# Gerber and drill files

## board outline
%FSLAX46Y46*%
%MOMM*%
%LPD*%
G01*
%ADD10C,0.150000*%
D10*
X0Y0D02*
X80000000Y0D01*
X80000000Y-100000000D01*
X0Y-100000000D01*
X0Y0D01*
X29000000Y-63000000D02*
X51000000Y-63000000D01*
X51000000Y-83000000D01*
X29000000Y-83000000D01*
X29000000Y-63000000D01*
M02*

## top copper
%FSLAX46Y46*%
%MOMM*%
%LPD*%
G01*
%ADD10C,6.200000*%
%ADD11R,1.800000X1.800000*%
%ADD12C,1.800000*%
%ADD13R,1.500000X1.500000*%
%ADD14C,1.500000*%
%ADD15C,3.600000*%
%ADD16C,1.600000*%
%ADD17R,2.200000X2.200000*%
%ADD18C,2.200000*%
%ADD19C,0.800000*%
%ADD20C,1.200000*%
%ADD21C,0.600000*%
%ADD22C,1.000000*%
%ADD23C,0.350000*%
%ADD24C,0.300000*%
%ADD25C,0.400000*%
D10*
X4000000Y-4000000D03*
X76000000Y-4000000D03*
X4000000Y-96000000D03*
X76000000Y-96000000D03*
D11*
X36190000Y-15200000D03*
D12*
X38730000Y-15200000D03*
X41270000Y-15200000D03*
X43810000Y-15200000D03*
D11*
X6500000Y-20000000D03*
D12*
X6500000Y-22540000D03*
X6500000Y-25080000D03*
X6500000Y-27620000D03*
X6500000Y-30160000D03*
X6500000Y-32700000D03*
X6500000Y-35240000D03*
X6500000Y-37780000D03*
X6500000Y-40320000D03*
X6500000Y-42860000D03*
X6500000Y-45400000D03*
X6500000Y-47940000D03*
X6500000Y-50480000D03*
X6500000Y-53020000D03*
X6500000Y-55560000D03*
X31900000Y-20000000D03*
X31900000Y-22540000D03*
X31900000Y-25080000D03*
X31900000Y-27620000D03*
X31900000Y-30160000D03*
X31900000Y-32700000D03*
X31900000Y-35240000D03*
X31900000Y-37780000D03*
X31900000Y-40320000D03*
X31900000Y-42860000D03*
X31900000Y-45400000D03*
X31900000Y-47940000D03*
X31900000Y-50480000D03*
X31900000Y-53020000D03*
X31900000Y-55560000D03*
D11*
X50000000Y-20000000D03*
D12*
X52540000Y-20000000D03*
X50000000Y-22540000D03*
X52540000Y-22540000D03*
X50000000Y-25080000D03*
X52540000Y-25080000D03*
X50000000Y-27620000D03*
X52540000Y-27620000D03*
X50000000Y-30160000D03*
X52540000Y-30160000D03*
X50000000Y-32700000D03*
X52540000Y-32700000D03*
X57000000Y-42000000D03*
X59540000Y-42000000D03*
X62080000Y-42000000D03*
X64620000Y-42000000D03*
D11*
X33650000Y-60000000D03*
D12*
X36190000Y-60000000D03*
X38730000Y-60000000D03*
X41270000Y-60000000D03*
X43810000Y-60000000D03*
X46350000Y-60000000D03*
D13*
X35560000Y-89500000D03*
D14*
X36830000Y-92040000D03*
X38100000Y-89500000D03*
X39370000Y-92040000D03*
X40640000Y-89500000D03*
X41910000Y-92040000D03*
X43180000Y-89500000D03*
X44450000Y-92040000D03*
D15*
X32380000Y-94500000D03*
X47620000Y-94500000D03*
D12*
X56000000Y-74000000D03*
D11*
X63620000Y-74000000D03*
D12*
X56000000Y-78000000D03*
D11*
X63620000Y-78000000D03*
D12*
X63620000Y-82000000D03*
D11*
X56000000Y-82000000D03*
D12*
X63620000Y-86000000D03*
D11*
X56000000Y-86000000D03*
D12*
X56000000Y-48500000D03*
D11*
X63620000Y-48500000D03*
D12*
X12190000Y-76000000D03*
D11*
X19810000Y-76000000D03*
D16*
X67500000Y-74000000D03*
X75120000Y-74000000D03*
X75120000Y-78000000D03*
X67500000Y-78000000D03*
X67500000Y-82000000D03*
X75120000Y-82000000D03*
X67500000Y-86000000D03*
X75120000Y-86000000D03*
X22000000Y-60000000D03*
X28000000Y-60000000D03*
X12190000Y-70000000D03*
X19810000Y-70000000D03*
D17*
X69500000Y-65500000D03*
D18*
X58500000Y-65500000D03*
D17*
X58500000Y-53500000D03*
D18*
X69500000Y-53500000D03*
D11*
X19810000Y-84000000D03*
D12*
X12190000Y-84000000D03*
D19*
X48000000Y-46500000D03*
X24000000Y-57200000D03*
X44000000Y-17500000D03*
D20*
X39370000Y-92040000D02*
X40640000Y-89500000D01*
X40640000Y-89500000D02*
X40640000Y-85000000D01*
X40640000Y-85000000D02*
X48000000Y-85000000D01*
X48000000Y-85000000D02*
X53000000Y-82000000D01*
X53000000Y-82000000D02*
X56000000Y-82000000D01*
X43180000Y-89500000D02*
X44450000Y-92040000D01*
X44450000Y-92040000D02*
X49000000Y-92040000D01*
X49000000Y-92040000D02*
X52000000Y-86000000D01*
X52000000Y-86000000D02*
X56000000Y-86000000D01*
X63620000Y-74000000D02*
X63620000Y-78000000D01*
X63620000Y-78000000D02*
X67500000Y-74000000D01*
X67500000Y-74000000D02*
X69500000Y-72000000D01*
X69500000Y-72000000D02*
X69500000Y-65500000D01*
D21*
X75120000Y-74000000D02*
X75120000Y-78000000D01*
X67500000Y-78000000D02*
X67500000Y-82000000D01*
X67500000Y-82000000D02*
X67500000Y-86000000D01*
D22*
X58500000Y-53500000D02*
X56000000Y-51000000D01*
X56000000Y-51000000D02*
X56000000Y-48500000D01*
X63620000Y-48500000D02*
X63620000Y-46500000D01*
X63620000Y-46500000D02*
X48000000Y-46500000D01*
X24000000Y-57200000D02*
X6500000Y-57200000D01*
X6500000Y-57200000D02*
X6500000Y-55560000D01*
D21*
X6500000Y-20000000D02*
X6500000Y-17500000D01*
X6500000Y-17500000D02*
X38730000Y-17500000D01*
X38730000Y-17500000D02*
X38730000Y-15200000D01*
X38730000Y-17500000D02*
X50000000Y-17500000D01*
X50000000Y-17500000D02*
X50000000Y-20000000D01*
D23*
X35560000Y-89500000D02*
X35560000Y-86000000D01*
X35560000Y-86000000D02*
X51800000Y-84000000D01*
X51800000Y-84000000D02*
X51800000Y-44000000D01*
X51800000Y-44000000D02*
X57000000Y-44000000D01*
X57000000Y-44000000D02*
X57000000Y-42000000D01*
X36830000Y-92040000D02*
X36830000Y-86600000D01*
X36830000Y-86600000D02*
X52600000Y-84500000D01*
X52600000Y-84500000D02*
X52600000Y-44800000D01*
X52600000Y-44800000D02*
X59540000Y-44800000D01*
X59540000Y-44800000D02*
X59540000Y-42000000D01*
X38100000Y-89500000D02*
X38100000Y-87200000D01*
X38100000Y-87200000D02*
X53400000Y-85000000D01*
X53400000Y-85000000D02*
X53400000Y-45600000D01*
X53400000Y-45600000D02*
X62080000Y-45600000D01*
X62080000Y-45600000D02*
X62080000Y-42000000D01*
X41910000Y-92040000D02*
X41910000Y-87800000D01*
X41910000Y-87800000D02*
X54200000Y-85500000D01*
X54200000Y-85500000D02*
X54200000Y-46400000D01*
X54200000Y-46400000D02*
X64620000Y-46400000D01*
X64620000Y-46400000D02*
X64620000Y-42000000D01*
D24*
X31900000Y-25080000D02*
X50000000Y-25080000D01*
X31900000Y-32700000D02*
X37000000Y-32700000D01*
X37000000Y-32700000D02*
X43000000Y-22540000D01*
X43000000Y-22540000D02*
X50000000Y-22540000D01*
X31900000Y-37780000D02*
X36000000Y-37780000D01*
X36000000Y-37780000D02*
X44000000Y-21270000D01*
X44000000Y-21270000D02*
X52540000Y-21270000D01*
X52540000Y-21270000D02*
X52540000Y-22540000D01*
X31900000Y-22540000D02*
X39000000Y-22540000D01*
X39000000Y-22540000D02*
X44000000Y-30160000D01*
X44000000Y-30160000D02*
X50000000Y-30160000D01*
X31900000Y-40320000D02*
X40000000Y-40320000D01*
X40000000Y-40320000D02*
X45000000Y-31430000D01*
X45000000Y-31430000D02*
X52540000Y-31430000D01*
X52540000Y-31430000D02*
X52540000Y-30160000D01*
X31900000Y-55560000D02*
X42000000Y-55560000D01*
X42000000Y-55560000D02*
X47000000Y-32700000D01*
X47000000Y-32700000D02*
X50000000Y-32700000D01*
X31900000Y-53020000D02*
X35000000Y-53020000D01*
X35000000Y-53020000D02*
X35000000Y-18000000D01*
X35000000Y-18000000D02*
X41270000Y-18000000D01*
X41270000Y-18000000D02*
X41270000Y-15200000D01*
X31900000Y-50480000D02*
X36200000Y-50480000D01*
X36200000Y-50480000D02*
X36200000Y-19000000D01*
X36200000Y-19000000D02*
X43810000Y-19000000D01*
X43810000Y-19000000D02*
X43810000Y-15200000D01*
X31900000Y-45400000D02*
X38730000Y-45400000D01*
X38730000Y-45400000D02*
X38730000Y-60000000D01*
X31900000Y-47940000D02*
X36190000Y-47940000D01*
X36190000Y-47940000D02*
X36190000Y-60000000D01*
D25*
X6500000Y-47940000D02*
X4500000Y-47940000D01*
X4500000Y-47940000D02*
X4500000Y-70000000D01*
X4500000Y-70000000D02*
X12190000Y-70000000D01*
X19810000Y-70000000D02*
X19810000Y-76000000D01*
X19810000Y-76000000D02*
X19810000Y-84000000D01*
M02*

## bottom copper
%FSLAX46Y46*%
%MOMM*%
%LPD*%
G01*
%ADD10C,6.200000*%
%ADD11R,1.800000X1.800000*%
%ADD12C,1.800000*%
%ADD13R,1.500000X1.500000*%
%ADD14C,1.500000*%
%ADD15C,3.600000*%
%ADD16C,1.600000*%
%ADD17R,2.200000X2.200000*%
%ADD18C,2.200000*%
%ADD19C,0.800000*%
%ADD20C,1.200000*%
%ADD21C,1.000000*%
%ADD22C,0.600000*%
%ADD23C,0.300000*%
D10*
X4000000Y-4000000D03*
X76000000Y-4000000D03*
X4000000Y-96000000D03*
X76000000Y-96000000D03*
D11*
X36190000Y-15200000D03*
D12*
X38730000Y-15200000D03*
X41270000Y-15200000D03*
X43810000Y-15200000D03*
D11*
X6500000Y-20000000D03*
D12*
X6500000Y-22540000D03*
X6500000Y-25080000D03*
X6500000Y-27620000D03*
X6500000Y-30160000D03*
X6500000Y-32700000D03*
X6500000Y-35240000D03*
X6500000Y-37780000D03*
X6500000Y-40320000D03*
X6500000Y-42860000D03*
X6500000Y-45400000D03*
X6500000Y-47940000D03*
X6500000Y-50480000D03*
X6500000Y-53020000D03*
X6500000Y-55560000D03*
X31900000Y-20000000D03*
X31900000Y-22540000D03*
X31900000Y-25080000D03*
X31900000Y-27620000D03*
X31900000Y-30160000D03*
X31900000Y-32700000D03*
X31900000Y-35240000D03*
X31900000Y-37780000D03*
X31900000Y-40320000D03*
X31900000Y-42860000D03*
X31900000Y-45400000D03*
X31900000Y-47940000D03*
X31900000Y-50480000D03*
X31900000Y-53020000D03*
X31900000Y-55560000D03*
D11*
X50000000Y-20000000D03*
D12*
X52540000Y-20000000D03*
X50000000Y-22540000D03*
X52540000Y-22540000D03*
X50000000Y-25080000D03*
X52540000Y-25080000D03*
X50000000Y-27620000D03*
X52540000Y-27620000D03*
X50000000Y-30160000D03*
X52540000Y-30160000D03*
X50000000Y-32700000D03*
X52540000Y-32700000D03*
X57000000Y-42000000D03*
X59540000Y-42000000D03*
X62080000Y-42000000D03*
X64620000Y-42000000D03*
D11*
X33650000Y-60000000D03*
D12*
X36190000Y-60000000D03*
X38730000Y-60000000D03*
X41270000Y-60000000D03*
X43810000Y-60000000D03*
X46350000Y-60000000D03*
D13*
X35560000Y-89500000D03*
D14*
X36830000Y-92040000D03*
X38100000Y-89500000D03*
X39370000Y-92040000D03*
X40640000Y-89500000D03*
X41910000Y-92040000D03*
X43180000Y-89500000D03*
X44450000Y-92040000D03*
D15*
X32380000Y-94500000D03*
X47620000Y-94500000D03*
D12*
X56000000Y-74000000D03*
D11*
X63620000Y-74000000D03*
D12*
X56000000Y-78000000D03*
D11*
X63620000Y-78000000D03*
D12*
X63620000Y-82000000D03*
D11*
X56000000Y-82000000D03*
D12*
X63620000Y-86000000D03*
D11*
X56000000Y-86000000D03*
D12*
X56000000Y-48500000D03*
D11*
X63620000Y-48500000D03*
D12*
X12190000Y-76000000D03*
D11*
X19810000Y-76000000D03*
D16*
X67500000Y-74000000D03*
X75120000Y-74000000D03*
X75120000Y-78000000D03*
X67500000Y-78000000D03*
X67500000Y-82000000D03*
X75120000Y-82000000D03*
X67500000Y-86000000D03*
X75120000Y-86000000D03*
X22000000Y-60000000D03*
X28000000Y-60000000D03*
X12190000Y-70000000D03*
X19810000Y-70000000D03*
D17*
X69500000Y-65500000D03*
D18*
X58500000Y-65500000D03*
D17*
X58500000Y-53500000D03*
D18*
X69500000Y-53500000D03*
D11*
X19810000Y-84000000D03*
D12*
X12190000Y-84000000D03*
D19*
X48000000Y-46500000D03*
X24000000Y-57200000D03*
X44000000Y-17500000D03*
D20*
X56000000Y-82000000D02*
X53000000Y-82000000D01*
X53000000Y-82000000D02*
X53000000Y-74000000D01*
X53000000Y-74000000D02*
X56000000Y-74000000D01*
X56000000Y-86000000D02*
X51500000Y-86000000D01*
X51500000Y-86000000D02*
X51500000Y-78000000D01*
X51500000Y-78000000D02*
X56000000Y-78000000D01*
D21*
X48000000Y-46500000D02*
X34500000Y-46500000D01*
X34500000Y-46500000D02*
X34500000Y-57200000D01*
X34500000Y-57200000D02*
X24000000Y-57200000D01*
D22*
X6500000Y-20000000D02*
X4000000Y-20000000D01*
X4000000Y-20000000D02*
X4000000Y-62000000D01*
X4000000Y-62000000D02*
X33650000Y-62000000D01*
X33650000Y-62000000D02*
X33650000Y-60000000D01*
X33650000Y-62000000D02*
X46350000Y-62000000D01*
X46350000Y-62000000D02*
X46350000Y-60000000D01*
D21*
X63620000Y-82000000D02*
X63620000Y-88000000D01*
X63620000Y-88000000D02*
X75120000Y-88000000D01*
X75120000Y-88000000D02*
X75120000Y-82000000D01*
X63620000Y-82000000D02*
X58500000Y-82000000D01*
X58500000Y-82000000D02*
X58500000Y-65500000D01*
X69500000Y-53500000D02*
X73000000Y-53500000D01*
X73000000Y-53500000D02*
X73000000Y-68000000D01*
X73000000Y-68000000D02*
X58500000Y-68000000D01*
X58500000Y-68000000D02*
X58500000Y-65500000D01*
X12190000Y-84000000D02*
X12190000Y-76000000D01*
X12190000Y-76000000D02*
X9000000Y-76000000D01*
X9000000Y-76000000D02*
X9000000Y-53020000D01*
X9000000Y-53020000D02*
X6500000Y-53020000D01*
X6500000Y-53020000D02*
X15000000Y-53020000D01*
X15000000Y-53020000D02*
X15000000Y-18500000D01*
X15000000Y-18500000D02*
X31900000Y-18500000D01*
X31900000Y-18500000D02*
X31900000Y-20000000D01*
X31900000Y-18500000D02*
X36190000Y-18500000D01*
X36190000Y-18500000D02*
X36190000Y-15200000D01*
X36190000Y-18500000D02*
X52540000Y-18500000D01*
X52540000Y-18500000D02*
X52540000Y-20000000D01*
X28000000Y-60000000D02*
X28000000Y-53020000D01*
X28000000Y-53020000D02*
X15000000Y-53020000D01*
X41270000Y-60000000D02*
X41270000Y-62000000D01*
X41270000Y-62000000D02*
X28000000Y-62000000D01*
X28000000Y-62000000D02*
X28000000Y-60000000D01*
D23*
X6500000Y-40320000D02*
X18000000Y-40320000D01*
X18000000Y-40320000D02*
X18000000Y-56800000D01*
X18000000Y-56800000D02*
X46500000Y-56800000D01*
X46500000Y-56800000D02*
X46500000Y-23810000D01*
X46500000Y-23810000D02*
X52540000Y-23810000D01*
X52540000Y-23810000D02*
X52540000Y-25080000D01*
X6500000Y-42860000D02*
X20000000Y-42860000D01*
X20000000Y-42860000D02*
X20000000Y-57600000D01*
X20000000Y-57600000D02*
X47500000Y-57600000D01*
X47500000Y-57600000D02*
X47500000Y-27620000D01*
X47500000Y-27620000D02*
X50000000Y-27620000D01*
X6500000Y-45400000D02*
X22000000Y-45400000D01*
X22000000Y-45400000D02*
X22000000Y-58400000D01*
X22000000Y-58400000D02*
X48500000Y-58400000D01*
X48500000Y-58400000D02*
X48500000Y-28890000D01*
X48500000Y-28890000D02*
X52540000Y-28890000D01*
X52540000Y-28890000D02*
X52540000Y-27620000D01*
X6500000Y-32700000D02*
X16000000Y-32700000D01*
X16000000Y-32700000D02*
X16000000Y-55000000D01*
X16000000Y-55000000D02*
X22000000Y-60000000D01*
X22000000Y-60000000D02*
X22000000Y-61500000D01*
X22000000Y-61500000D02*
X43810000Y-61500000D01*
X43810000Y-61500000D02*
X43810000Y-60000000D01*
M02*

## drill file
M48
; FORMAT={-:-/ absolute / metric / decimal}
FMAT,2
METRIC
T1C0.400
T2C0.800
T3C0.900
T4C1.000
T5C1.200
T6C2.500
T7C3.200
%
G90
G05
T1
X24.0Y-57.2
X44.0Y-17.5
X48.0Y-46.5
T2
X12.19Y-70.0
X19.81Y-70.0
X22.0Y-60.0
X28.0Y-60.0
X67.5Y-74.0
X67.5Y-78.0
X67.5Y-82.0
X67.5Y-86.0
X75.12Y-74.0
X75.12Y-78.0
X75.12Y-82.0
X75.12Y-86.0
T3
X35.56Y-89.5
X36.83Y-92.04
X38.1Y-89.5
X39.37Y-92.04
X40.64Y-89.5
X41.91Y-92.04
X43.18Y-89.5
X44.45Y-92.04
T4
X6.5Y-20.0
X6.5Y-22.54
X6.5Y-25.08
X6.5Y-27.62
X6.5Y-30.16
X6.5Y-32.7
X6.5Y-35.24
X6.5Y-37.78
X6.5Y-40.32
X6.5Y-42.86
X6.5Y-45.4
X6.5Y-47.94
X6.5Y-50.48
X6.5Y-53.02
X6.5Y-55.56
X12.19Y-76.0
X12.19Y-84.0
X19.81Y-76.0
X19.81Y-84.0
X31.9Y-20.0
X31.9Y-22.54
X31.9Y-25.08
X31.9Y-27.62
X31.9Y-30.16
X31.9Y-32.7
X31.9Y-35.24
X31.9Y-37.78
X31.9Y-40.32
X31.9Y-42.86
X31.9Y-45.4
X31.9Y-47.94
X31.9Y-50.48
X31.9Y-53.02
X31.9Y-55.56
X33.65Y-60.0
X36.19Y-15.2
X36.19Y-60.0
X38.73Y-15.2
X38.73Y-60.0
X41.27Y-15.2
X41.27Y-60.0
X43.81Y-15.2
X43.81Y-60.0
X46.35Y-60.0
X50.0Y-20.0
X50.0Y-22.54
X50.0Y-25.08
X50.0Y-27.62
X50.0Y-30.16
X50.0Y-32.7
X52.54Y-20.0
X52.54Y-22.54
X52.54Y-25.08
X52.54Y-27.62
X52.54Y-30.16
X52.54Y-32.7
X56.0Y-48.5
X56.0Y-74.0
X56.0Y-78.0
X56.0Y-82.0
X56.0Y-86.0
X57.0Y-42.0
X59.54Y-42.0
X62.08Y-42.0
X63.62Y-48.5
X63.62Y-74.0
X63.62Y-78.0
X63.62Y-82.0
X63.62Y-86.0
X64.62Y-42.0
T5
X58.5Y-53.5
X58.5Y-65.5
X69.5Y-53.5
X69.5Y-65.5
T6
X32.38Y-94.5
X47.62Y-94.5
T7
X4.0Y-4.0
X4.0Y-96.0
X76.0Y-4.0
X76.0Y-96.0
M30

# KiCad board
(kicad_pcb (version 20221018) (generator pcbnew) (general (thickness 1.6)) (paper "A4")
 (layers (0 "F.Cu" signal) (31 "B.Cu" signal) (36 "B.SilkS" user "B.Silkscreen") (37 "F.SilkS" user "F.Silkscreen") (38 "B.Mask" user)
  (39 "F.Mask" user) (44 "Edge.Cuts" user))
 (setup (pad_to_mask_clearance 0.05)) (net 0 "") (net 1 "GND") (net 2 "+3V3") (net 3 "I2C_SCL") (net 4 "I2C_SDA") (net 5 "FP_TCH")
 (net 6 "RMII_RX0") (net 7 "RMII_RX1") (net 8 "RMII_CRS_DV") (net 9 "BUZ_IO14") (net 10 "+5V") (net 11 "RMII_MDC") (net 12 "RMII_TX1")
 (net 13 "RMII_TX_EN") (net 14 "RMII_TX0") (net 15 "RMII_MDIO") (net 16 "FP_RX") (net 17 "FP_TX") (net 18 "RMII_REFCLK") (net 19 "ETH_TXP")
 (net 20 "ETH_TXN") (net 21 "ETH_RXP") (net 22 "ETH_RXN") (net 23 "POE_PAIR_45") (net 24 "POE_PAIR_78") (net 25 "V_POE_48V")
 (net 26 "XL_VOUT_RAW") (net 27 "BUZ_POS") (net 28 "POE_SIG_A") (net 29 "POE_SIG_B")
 (gr_rect (start 0 0) (end 80.0 100.0) (layer "Edge.Cuts") (width 0.15))
 (gr_rect (start 29.0 63.0) (end 51.0 83.0) (layer "Edge.Cuts") (width 0.15))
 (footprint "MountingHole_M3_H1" (layer "F.Cu") (at 4.0 4.0)
  (pad "H1" thru_hole circle (at 0 0) (size 6.2 6.2) (drill 3.2) (layers "*.Cu" "*.Mask") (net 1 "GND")))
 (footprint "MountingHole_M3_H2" (layer "F.Cu") (at 76.0 4.0)
  (pad "H2" thru_hole circle (at 0 0) (size 6.2 6.2) (drill 3.2) (layers "*.Cu" "*.Mask") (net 1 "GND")))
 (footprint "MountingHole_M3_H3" (layer "F.Cu") (at 4.0 96.0)
  (pad "H3" thru_hole circle (at 0 0) (size 6.2 6.2) (drill 3.2) (layers "*.Cu" "*.Mask") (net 1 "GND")))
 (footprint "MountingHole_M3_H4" (layer "F.Cu") (at 76.0 96.0)
  (pad "H4" thru_hole circle (at 0 0) (size 6.2 6.2) (drill 3.2) (layers "*.Cu" "*.Mask") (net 1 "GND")))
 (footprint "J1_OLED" (layer "F.Cu") (at 36.19 15.20)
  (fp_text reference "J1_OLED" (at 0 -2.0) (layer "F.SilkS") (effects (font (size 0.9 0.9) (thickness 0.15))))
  (pad "1" thru_hole rect (at 0.00 0.00) (size 1.80 1.80) (drill 1.00) (layers "*.Cu" "*.Mask") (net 1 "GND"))
  (pad "2" thru_hole circle (at 2.54 0.00) (size 1.80 1.80) (drill 1.00) (layers "*.Cu" "*.Mask") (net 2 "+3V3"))
  (pad "3" thru_hole circle (at 5.08 0.00) (size 1.80 1.80) (drill 1.00) (layers "*.Cu" "*.Mask") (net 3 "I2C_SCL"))
  (pad "4" thru_hole circle (at 7.62 0.00) (size 1.80 1.80) (drill 1.00) (layers "*.Cu" "*.Mask") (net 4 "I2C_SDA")))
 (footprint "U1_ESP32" (layer "F.Cu") (at 6.50 20.00)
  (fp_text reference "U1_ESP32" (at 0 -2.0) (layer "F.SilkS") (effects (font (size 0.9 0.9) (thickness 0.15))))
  (pad "1" thru_hole rect (at 0.00 0.00) (size 1.80 1.80) (drill 1.00) (layers "*.Cu" "*.Mask") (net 2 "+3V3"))
  (pad "2" thru_hole circle (at 0.00 2.54) (size 1.80 1.80) (drill 1.00) (layers "*.Cu" "*.Mask"))
  (pad "3" thru_hole circle (at 0.00 5.08) (size 1.80 1.80) (drill 1.00) (layers "*.Cu" "*.Mask"))
  (pad "4" thru_hole circle (at 0.00 7.62) (size 1.80 1.80) (drill 1.00) (layers "*.Cu" "*.Mask"))
  (pad "5" thru_hole circle (at 0.00 10.16) (size 1.80 1.80) (drill 1.00) (layers "*.Cu" "*.Mask"))
  (pad "6" thru_hole circle (at 0.00 12.70) (size 1.80 1.80) (drill 1.00) (layers "*.Cu" "*.Mask") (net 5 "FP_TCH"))
  (pad "7" thru_hole circle (at 0.00 15.24) (size 1.80 1.80) (drill 1.00) (layers "*.Cu" "*.Mask"))
  (pad "8" thru_hole circle (at 0.00 17.78) (size 1.80 1.80) (drill 1.00) (layers "*.Cu" "*.Mask"))
  (pad "9" thru_hole circle (at 0.00 20.32) (size 1.80 1.80) (drill 1.00) (layers "*.Cu" "*.Mask") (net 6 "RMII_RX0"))
  (pad "10" thru_hole circle (at 0.00 22.86) (size 1.80 1.80) (drill 1.00) (layers "*.Cu" "*.Mask") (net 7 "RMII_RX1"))
  (pad "11" thru_hole circle (at 0.00 25.40) (size 1.80 1.80) (drill 1.00) (layers "*.Cu" "*.Mask") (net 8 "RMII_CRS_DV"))
  (pad "12" thru_hole circle (at 0.00 27.94) (size 1.80 1.80) (drill 1.00) (layers "*.Cu" "*.Mask") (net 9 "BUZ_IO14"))
  (pad "13" thru_hole circle (at 0.00 30.48) (size 1.80 1.80) (drill 1.00) (layers "*.Cu" "*.Mask"))
  (pad "14" thru_hole circle (at 0.00 33.02) (size 1.80 1.80) (drill 1.00) (layers "*.Cu" "*.Mask") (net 1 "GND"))
  (pad "15" thru_hole circle (at 0.00 35.56) (size 1.80 1.80) (drill 1.00) (layers "*.Cu" "*.Mask") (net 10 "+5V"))
  (pad "30" thru_hole circle (at 25.40 0.00) (size 1.80 1.80) (drill 1.00) (layers "*.Cu" "*.Mask") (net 1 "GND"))
  (pad "29" thru_hole circle (at 25.40 2.54) (size 1.80 1.80) (drill 1.00) (layers "*.Cu" "*.Mask") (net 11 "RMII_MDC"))
  (pad "28" thru_hole circle (at 25.40 5.08) (size 1.80 1.80) (drill 1.00) (layers "*.Cu" "*.Mask") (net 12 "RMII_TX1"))
  (pad "27" thru_hole circle (at 25.40 7.62) (size 1.80 1.80) (drill 1.00) (layers "*.Cu" "*.Mask"))
  (pad "26" thru_hole circle (at 25.40 10.16) (size 1.80 1.80) (drill 1.00) (layers "*.Cu" "*.Mask"))
  (pad "25" thru_hole circle (at 25.40 12.70) (size 1.80 1.80) (drill 1.00) (layers "*.Cu" "*.Mask") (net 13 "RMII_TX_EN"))
  (pad "24" thru_hole circle (at 25.40 15.24) (size 1.80 1.80) (drill 1.00) (layers "*.Cu" "*.Mask") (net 1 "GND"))
  (pad "23" thru_hole circle (at 25.40 17.78) (size 1.80 1.80) (drill 1.00) (layers "*.Cu" "*.Mask") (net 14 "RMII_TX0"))
  (pad "22" thru_hole circle (at 25.40 20.32) (size 1.80 1.80) (drill 1.00) (layers "*.Cu" "*.Mask") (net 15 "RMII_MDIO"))
  (pad "21" thru_hole circle (at 25.40 22.86) (size 1.80 1.80) (drill 1.00) (layers "*.Cu" "*.Mask"))
  (pad "20" thru_hole circle (at 25.40 25.40) (size 1.80 1.80) (drill 1.00) (layers "*.Cu" "*.Mask") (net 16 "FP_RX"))
  (pad "19" thru_hole circle (at 25.40 27.94) (size 1.80 1.80) (drill 1.00) (layers "*.Cu" "*.Mask") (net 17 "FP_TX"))
  (pad "18" thru_hole circle (at 25.40 30.48) (size 1.80 1.80) (drill 1.00) (layers "*.Cu" "*.Mask") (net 4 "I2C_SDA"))
  (pad "17" thru_hole circle (at 25.40 33.02) (size 1.80 1.80) (drill 1.00) (layers "*.Cu" "*.Mask") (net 3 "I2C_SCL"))
  (pad "16" thru_hole circle (at 25.40 35.56) (size 1.80 1.80) (drill 1.00) (layers "*.Cu" "*.Mask") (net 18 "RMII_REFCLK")))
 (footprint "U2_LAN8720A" (layer "F.Cu") (at 50.00 20.00)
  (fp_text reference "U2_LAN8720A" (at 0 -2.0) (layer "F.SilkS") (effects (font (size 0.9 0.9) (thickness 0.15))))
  (pad "1" thru_hole rect (at 0.00 0.00) (size 1.80 1.80) (drill 1.00) (layers "*.Cu" "*.Mask") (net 2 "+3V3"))
  (pad "2" thru_hole circle (at 2.54 0.00) (size 1.80 1.80) (drill 1.00) (layers "*.Cu" "*.Mask") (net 1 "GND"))
  (pad "3" thru_hole circle (at 0.00 2.54) (size 1.80 1.80) (drill 1.00) (layers "*.Cu" "*.Mask") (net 13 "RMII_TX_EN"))
  (pad "4" thru_hole circle (at 2.54 2.54) (size 1.80 1.80) (drill 1.00) (layers "*.Cu" "*.Mask") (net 14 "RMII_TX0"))
  (pad "5" thru_hole circle (at 0.00 5.08) (size 1.80 1.80) (drill 1.00) (layers "*.Cu" "*.Mask") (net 12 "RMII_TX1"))
  (pad "6" thru_hole circle (at 2.54 5.08) (size 1.80 1.80) (drill 1.00) (layers "*.Cu" "*.Mask") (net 6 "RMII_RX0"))
  (pad "7" thru_hole circle (at 0.00 7.62) (size 1.80 1.80) (drill 1.00) (layers "*.Cu" "*.Mask") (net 7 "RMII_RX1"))
  (pad "8" thru_hole circle (at 2.54 7.62) (size 1.80 1.80) (drill 1.00) (layers "*.Cu" "*.Mask") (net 8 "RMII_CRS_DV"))
  (pad "9" thru_hole circle (at 0.00 10.16) (size 1.80 1.80) (drill 1.00) (layers "*.Cu" "*.Mask") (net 11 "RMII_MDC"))
  (pad "10" thru_hole circle (at 2.54 10.16) (size 1.80 1.80) (drill 1.00) (layers "*.Cu" "*.Mask") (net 15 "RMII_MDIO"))
  (pad "11" thru_hole circle (at 0.00 12.70) (size 1.80 1.80) (drill 1.00) (layers "*.Cu" "*.Mask") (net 18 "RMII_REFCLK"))
  (pad "12" thru_hole circle (at 2.54 12.70) (size 1.80 1.80) (drill 1.00) (layers "*.Cu" "*.Mask") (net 2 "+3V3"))
  (pad "E1" thru_hole circle (at 7.00 22.00) (size 1.80 1.80) (drill 1.00) (layers "*.Cu" "*.Mask") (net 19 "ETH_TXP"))
  (pad "E2" thru_hole circle (at 9.54 22.00) (size 1.80 1.80) (drill 1.00) (layers "*.Cu" "*.Mask") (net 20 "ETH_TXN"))
  (pad "E3" thru_hole circle (at 12.08 22.00) (size 1.80 1.80) (drill 1.00) (layers "*.Cu" "*.Mask") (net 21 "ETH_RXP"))
  (pad "E6" thru_hole circle (at 14.62 22.00) (size 1.80 1.80) (drill 1.00) (layers "*.Cu" "*.Mask") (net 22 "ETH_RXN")))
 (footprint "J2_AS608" (layer "F.Cu") (at 33.65 60.00)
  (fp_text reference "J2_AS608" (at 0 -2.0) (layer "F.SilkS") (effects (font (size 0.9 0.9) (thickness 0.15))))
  (pad "1" thru_hole rect (at 0.00 0.00) (size 1.80 1.80) (drill 1.00) (layers "*.Cu" "*.Mask") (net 2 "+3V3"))
  (pad "2" thru_hole circle (at 2.54 0.00) (size 1.80 1.80) (drill 1.00) (layers "*.Cu" "*.Mask") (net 17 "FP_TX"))
  (pad "3" thru_hole circle (at 5.08 0.00) (size 1.80 1.80) (drill 1.00) (layers "*.Cu" "*.Mask") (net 16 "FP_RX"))
  (pad "4" thru_hole circle (at 7.62 0.00) (size 1.80 1.80) (drill 1.00) (layers "*.Cu" "*.Mask") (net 1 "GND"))
  (pad "5" thru_hole circle (at 10.16 0.00) (size 1.80 1.80) (drill 1.00) (layers "*.Cu" "*.Mask") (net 5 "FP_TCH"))
  (pad "6" thru_hole circle (at 12.70 0.00) (size 1.80 1.80) (drill 1.00) (layers "*.Cu" "*.Mask") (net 2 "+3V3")))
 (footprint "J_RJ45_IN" (layer "F.Cu") (at 35.56 89.50)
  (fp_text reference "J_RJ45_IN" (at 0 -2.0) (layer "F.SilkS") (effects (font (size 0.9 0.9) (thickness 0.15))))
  (pad "1" thru_hole rect (at 0.00 0.00) (size 1.50 1.50) (drill 0.90) (layers "*.Cu" "*.Mask") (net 19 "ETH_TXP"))
  (pad "2" thru_hole circle (at 1.27 2.54) (size 1.50 1.50) (drill 0.90) (layers "*.Cu" "*.Mask") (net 20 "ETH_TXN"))
  (pad "3" thru_hole circle (at 2.54 0.00) (size 1.50 1.50) (drill 0.90) (layers "*.Cu" "*.Mask") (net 21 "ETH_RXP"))
  (pad "4" thru_hole circle (at 3.81 2.54) (size 1.50 1.50) (drill 0.90) (layers "*.Cu" "*.Mask") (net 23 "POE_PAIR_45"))
  (pad "5" thru_hole circle (at 5.08 0.00) (size 1.50 1.50) (drill 0.90) (layers "*.Cu" "*.Mask") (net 23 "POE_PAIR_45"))
  (pad "6" thru_hole circle (at 6.35 2.54) (size 1.50 1.50) (drill 0.90) (layers "*.Cu" "*.Mask") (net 22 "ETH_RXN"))
  (pad "7" thru_hole circle (at 7.62 0.00) (size 1.50 1.50) (drill 0.90) (layers "*.Cu" "*.Mask") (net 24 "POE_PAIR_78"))
  (pad "8" thru_hole circle (at 8.89 2.54) (size 1.50 1.50) (drill 0.90) (layers "*.Cu" "*.Mask") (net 24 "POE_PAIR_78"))
  (pad "M1" thru_hole circle (at -3.18 5.00) (size 3.60 3.60) (drill 2.50) (layers "*.Cu" "*.Mask"))
  (pad "M2" thru_hole circle (at 12.06 5.00) (size 3.60 3.60) (drill 2.50) (layers "*.Cu" "*.Mask")))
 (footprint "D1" (layer "F.Cu") (at 56.00 74.00)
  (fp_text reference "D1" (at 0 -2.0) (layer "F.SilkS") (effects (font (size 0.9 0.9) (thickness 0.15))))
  (pad "A" thru_hole circle (at 0.00 0.00) (size 1.80 1.80) (drill 1.00) (layers "*.Cu" "*.Mask") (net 23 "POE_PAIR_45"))
  (pad "K" thru_hole rect (at 7.62 0.00) (size 1.80 1.80) (drill 1.00) (layers "*.Cu" "*.Mask") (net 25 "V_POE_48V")))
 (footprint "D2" (layer "F.Cu") (at 56.00 78.00)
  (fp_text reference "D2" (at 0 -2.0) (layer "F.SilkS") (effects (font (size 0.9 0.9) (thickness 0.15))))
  (pad "A" thru_hole circle (at 0.00 0.00) (size 1.80 1.80) (drill 1.00) (layers "*.Cu" "*.Mask") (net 24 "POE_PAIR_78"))
  (pad "K" thru_hole rect (at 7.62 0.00) (size 1.80 1.80) (drill 1.00) (layers "*.Cu" "*.Mask") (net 25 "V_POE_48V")))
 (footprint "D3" (layer "F.Cu") (at 63.62 82.00)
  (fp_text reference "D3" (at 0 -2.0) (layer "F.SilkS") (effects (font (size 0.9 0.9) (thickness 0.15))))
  (pad "A" thru_hole circle (at 0.00 0.00) (size 1.80 1.80) (drill 1.00) (layers "*.Cu" "*.Mask") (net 1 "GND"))
  (pad "K" thru_hole rect (at -7.62 0.00) (size 1.80 1.80) (drill 1.00) (layers "*.Cu" "*.Mask") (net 23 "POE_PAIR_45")))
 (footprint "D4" (layer "F.Cu") (at 63.62 86.00)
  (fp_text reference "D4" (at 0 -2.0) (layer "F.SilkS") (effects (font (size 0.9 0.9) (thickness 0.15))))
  (pad "A" thru_hole circle (at 0.00 0.00) (size 1.80 1.80) (drill 1.00) (layers "*.Cu" "*.Mask") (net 1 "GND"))
  (pad "K" thru_hole rect (at -7.62 0.00) (size 1.80 1.80) (drill 1.00) (layers "*.Cu" "*.Mask") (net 24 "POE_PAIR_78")))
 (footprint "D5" (layer "F.Cu") (at 56.00 48.50)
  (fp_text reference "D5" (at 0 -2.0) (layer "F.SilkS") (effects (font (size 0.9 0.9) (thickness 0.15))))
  (pad "A" thru_hole circle (at 0.00 0.00) (size 1.80 1.80) (drill 1.00) (layers "*.Cu" "*.Mask") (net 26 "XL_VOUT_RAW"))
  (pad "K" thru_hole rect (at 7.62 0.00) (size 1.80 1.80) (drill 1.00) (layers "*.Cu" "*.Mask") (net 10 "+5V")))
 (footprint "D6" (layer "F.Cu") (at 12.19 76.00)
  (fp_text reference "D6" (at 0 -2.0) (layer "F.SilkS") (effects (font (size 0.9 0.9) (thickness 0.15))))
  (pad "A" thru_hole circle (at 0.00 0.00) (size 1.80 1.80) (drill 1.00) (layers "*.Cu" "*.Mask") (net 1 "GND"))
  (pad "K" thru_hole rect (at 7.62 0.00) (size 1.80 1.80) (drill 1.00) (layers "*.Cu" "*.Mask") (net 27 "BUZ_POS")))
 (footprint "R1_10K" (layer "F.Cu") (at 67.50 74.00)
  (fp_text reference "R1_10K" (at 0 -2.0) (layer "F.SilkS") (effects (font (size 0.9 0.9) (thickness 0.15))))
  (pad "1" thru_hole circle (at 0.00 0.00) (size 1.60 1.60) (drill 0.80) (layers "*.Cu" "*.Mask") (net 25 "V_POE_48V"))
  (pad "2" thru_hole circle (at 7.62 0.00) (size 1.60 1.60) (drill 0.80) (layers "*.Cu" "*.Mask") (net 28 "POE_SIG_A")))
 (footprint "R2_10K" (layer "F.Cu") (at 75.12 78.00)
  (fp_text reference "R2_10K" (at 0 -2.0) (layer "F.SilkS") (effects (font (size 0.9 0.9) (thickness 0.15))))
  (pad "1" thru_hole circle (at 0.00 0.00) (size 1.60 1.60) (drill 0.80) (layers "*.Cu" "*.Mask") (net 28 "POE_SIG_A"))
  (pad "2" thru_hole circle (at -7.62 0.00) (size 1.60 1.60) (drill 0.80) (layers "*.Cu" "*.Mask") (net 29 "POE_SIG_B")))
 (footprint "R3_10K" (layer "F.Cu") (at 67.50 82.00)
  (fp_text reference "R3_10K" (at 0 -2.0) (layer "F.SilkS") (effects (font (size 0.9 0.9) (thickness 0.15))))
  (pad "1" thru_hole circle (at 0.00 0.00) (size 1.60 1.60) (drill 0.80) (layers "*.Cu" "*.Mask") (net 29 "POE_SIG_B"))
  (pad "2" thru_hole circle (at 7.62 0.00) (size 1.60 1.60) (drill 0.80) (layers "*.Cu" "*.Mask") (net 1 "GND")))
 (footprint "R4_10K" (layer "F.Cu") (at 67.50 86.00)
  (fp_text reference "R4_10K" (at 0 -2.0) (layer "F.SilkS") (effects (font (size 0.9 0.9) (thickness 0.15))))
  (pad "1" thru_hole circle (at 0.00 0.00) (size 1.60 1.60) (drill 0.80) (layers "*.Cu" "*.Mask") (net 29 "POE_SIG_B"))
  (pad "2" thru_hole circle (at 7.62 0.00) (size 1.60 1.60) (drill 0.80) (layers "*.Cu" "*.Mask") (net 1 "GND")))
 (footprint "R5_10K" (layer "F.Cu") (at 22.00 60.00)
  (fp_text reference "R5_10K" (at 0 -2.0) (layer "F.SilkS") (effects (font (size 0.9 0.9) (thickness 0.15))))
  (pad "1" thru_hole circle (at 0.00 0.00) (size 1.60 1.60) (drill 0.80) (layers "*.Cu" "*.Mask") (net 5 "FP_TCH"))
  (pad "2" thru_hole circle (at 6.00 0.00) (size 1.60 1.60) (drill 0.80) (layers "*.Cu" "*.Mask") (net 1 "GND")))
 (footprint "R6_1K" (layer "F.Cu") (at 12.19 70.00)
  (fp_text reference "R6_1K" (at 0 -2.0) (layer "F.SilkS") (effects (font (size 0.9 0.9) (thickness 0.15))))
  (pad "1" thru_hole circle (at 0.00 0.00) (size 1.60 1.60) (drill 0.80) (layers "*.Cu" "*.Mask") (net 9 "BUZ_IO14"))
  (pad "2" thru_hole circle (at 7.62 0.00) (size 1.60 1.60) (drill 0.80) (layers "*.Cu" "*.Mask") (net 27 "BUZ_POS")))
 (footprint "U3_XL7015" (layer "F.Cu") (at 69.50 65.50)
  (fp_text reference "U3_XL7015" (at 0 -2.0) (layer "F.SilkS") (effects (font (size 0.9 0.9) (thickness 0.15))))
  (pad "VIN+" thru_hole rect (at 0.00 0.00) (size 2.20 2.20) (drill 1.20) (layers "*.Cu" "*.Mask") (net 25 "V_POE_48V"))
  (pad "VIN-" thru_hole circle (at -11.00 0.00) (size 2.20 2.20) (drill 1.20) (layers "*.Cu" "*.Mask") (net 1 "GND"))
  (pad "VOUT+" thru_hole rect (at -11.00 -12.00) (size 2.20 2.20) (drill 1.20) (layers "*.Cu" "*.Mask") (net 26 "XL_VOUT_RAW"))
  (pad "VOUT-" thru_hole circle (at 0.00 -12.00) (size 2.20 2.20) (drill 1.20) (layers "*.Cu" "*.Mask") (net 1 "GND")))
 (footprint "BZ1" (layer "F.Cu") (at 19.81 84.00)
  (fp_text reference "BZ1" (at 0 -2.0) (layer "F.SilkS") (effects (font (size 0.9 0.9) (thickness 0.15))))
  (pad "+" thru_hole rect (at 0.00 0.00) (size 1.80 1.80) (drill 1.00) (layers "*.Cu" "*.Mask") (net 27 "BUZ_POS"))
  (pad "-" thru_hole circle (at -7.62 0.00) (size 1.80 1.80) (drill 1.00) (layers "*.Cu" "*.Mask") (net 1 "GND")))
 (via (at 48.00 46.50) (size 0.8) (drill 0.4) (layers "F.Cu" "B.Cu") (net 10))
 (via (at 24.00 57.20) (size 0.8) (drill 0.4) (layers "F.Cu" "B.Cu") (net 10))
 (via (at 44.00 17.50) (size 0.8) (drill 0.4) (layers "F.Cu" "B.Cu") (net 2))
 (segment (start 39.37 92.04) (end 40.64 89.50) (width 1.20) (layer "F.Cu") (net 23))
 (segment (start 40.64 89.50) (end 40.64 85.00) (width 1.20) (layer "F.Cu") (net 23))
 (segment (start 40.64 85.00) (end 48.00 85.00) (width 1.20) (layer "F.Cu") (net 23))
 (segment (start 48.00 85.00) (end 53.00 82.00) (width 1.20) (layer "F.Cu") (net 23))
 (segment (start 53.00 82.00) (end 56.00 82.00) (width 1.20) (layer "F.Cu") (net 23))
 (segment (start 56.00 82.00) (end 53.00 82.00) (width 1.20) (layer "B.Cu") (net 23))
 (segment (start 53.00 82.00) (end 53.00 74.00) (width 1.20) (layer "B.Cu") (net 23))
 (segment (start 53.00 74.00) (end 56.00 74.00) (width 1.20) (layer "B.Cu") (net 23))
 (segment (start 43.18 89.50) (end 44.45 92.04) (width 1.20) (layer "F.Cu") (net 24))
 (segment (start 44.45 92.04) (end 49.00 92.04) (width 1.20) (layer "F.Cu") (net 24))
 (segment (start 49.00 92.04) (end 52.00 86.00) (width 1.20) (layer "F.Cu") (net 24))
 (segment (start 52.00 86.00) (end 56.00 86.00) (width 1.20) (layer "F.Cu") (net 24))
 (segment (start 56.00 86.00) (end 51.50 86.00) (width 1.20) (layer "B.Cu") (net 24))
 (segment (start 51.50 86.00) (end 51.50 78.00) (width 1.20) (layer "B.Cu") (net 24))
 (segment (start 51.50 78.00) (end 56.00 78.00) (width 1.20) (layer "B.Cu") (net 24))
 (segment (start 63.62 74.00) (end 63.62 78.00) (width 1.20) (layer "F.Cu") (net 25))
 (segment (start 63.62 78.00) (end 67.50 74.00) (width 1.20) (layer "F.Cu") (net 25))
 (segment (start 67.50 74.00) (end 69.50 72.00) (width 1.20) (layer "F.Cu") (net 25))
 (segment (start 69.50 72.00) (end 69.50 65.50) (width 1.20) (layer "F.Cu") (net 25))
 (segment (start 75.12 74.00) (end 75.12 78.00) (width 0.60) (layer "F.Cu") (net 28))
 (segment (start 67.50 78.00) (end 67.50 82.00) (width 0.60) (layer "F.Cu") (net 29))
 (segment (start 67.50 82.00) (end 67.50 86.00) (width 0.60) (layer "F.Cu") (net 29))
 (segment (start 58.50 53.50) (end 56.00 51.00) (width 1.00) (layer "F.Cu") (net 26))
 (segment (start 56.00 51.00) (end 56.00 48.50) (width 1.00) (layer "F.Cu") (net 26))
 (segment (start 63.62 48.50) (end 63.62 46.50) (width 1.00) (layer "F.Cu") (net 10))
 (segment (start 63.62 46.50) (end 48.00 46.50) (width 1.00) (layer "F.Cu") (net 10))
 (segment (start 48.00 46.50) (end 34.50 46.50) (width 1.00) (layer "B.Cu") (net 10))
 (segment (start 34.50 46.50) (end 34.50 57.20) (width 1.00) (layer "B.Cu") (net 10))
 (segment (start 34.50 57.20) (end 24.00 57.20) (width 1.00) (layer "B.Cu") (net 10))
 (segment (start 24.00 57.20) (end 6.50 57.20) (width 1.00) (layer "F.Cu") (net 10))
 (segment (start 6.50 57.20) (end 6.50 55.56) (width 1.00) (layer "F.Cu") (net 10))
 (segment (start 6.50 20.00) (end 6.50 17.50) (width 0.60) (layer "F.Cu") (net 2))
 (segment (start 6.50 17.50) (end 38.73 17.50) (width 0.60) (layer "F.Cu") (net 2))
 (segment (start 38.73 17.50) (end 38.73 15.20) (width 0.60) (layer "F.Cu") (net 2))
 (segment (start 38.73 17.50) (end 50.00 17.50) (width 0.60) (layer "F.Cu") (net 2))
 (segment (start 50.00 17.50) (end 50.00 20.00) (width 0.60) (layer "F.Cu") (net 2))
 (segment (start 6.50 20.00) (end 4.00 20.00) (width 0.60) (layer "B.Cu") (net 2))
 (segment (start 4.00 20.00) (end 4.00 62.00) (width 0.60) (layer "B.Cu") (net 2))
 (segment (start 4.00 62.00) (end 33.65 62.00) (width 0.60) (layer "B.Cu") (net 2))
 (segment (start 33.65 62.00) (end 33.65 60.00) (width 0.60) (layer "B.Cu") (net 2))
 (segment (start 33.65 62.00) (end 46.35 62.00) (width 0.60) (layer "B.Cu") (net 2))
 (segment (start 46.35 62.00) (end 46.35 60.00) (width 0.60) (layer "B.Cu") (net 2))
 (segment (start 63.62 82.00) (end 63.62 88.00) (width 1.00) (layer "B.Cu") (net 1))
 (segment (start 63.62 88.00) (end 75.12 88.00) (width 1.00) (layer "B.Cu") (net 1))
 (segment (start 75.12 88.00) (end 75.12 82.00) (width 1.00) (layer "B.Cu") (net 1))
 (segment (start 63.62 82.00) (end 58.50 82.00) (width 1.00) (layer "B.Cu") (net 1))
 (segment (start 58.50 82.00) (end 58.50 65.50) (width 1.00) (layer "B.Cu") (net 1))
 (segment (start 69.50 53.50) (end 73.00 53.50) (width 1.00) (layer "B.Cu") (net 1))
 (segment (start 73.00 53.50) (end 73.00 68.00) (width 1.00) (layer "B.Cu") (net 1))
 (segment (start 73.00 68.00) (end 58.50 68.00) (width 1.00) (layer "B.Cu") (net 1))
 (segment (start 58.50 68.00) (end 58.50 65.50) (width 1.00) (layer "B.Cu") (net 1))
 (segment (start 12.19 84.00) (end 12.19 76.00) (width 1.00) (layer "B.Cu") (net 1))
 (segment (start 12.19 76.00) (end 9.00 76.00) (width 1.00) (layer "B.Cu") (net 1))
 (segment (start 9.00 76.00) (end 9.00 53.02) (width 1.00) (layer "B.Cu") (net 1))
 (segment (start 9.00 53.02) (end 6.50 53.02) (width 1.00) (layer "B.Cu") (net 1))
 (segment (start 6.50 53.02) (end 15.00 53.02) (width 1.00) (layer "B.Cu") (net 1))
 (segment (start 15.00 53.02) (end 15.00 18.50) (width 1.00) (layer "B.Cu") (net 1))
 (segment (start 15.00 18.50) (end 31.90 18.50) (width 1.00) (layer "B.Cu") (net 1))
 (segment (start 31.90 18.50) (end 31.90 20.00) (width 1.00) (layer "B.Cu") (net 1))
 (segment (start 31.90 18.50) (end 36.19 18.50) (width 1.00) (layer "B.Cu") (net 1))
 (segment (start 36.19 18.50) (end 36.19 15.20) (width 1.00) (layer "B.Cu") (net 1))
 (segment (start 36.19 18.50) (end 52.54 18.50) (width 1.00) (layer "B.Cu") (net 1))
 (segment (start 52.54 18.50) (end 52.54 20.00) (width 1.00) (layer "B.Cu") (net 1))
 (segment (start 28.00 60.00) (end 28.00 53.02) (width 1.00) (layer "B.Cu") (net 1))
 (segment (start 28.00 53.02) (end 15.00 53.02) (width 1.00) (layer "B.Cu") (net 1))
 (segment (start 41.27 60.00) (end 41.27 62.00) (width 1.00) (layer "B.Cu") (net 1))
 (segment (start 41.27 62.00) (end 28.00 62.00) (width 1.00) (layer "B.Cu") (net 1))
 (segment (start 28.00 62.00) (end 28.00 60.00) (width 1.00) (layer "B.Cu") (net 1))
 (segment (start 35.56 89.50) (end 35.56 86.00) (width 0.35) (layer "F.Cu") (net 19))
 (segment (start 35.56 86.00) (end 51.80 84.00) (width 0.35) (layer "F.Cu") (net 19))
 (segment (start 51.80 84.00) (end 51.80 44.00) (width 0.35) (layer "F.Cu") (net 19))
 (segment (start 51.80 44.00) (end 57.00 44.00) (width 0.35) (layer "F.Cu") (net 19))
 (segment (start 57.00 44.00) (end 57.00 42.00) (width 0.35) (layer "F.Cu") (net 19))
 (segment (start 36.83 92.04) (end 36.83 86.60) (width 0.35) (layer "F.Cu") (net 20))
 (segment (start 36.83 86.60) (end 52.60 84.50) (width 0.35) (layer "F.Cu") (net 20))
 (segment (start 52.60 84.50) (end 52.60 44.80) (width 0.35) (layer "F.Cu") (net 20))
 (segment (start 52.60 44.80) (end 59.54 44.80) (width 0.35) (layer "F.Cu") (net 20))
 (segment (start 59.54 44.80) (end 59.54 42.00) (width 0.35) (layer "F.Cu") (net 20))
 (segment (start 38.10 89.50) (end 38.10 87.20) (width 0.35) (layer "F.Cu") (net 21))
 (segment (start 38.10 87.20) (end 53.40 85.00) (width 0.35) (layer "F.Cu") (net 21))
 (segment (start 53.40 85.00) (end 53.40 45.60) (width 0.35) (layer "F.Cu") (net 21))
 (segment (start 53.40 45.60) (end 62.08 45.60) (width 0.35) (layer "F.Cu") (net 21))
 (segment (start 62.08 45.60) (end 62.08 42.00) (width 0.35) (layer "F.Cu") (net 21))
 (segment (start 41.91 92.04) (end 41.91 87.80) (width 0.35) (layer "F.Cu") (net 22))
 (segment (start 41.91 87.80) (end 54.20 85.50) (width 0.35) (layer "F.Cu") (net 22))
 (segment (start 54.20 85.50) (end 54.20 46.40) (width 0.35) (layer "F.Cu") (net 22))
 (segment (start 54.20 46.40) (end 64.62 46.40) (width 0.35) (layer "F.Cu") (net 22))
 (segment (start 64.62 46.40) (end 64.62 42.00) (width 0.35) (layer "F.Cu") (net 22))
 (segment (start 31.90 25.08) (end 50.00 25.08) (width 0.30) (layer "F.Cu") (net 12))
 (segment (start 31.90 32.70) (end 37.00 32.70) (width 0.30) (layer "F.Cu") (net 13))
 (segment (start 37.00 32.70) (end 43.00 22.54) (width 0.30) (layer "F.Cu") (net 13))
 (segment (start 43.00 22.54) (end 50.00 22.54) (width 0.30) (layer "F.Cu") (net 13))
 (segment (start 31.90 37.78) (end 36.00 37.78) (width 0.30) (layer "F.Cu") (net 14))
 (segment (start 36.00 37.78) (end 44.00 21.27) (width 0.30) (layer "F.Cu") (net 14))
 (segment (start 44.00 21.27) (end 52.54 21.27) (width 0.30) (layer "F.Cu") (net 14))
 (segment (start 52.54 21.27) (end 52.54 22.54) (width 0.30) (layer "F.Cu") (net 14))
 (segment (start 31.90 22.54) (end 39.00 22.54) (width 0.30) (layer "F.Cu") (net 11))
 (segment (start 39.00 22.54) (end 44.00 30.16) (width 0.30) (layer "F.Cu") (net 11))
 (segment (start 44.00 30.16) (end 50.00 30.16) (width 0.30) (layer "F.Cu") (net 11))
 (segment (start 31.90 40.32) (end 40.00 40.32) (width 0.30) (layer "F.Cu") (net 15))
 (segment (start 40.00 40.32) (end 45.00 31.43) (width 0.30) (layer "F.Cu") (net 15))
 (segment (start 45.00 31.43) (end 52.54 31.43) (width 0.30) (layer "F.Cu") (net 15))
 (segment (start 52.54 31.43) (end 52.54 30.16) (width 0.30) (layer "F.Cu") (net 15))
 (segment (start 31.90 55.56) (end 42.00 55.56) (width 0.30) (layer "F.Cu") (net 18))
 (segment (start 42.00 55.56) (end 47.00 32.70) (width 0.30) (layer "F.Cu") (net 18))
 (segment (start 47.00 32.70) (end 50.00 32.70) (width 0.30) (layer "F.Cu") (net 18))
 (segment (start 6.50 40.32) (end 18.00 40.32) (width 0.30) (layer "B.Cu") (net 6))
 (segment (start 18.00 40.32) (end 18.00 56.80) (width 0.30) (layer "B.Cu") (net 6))
 (segment (start 18.00 56.80) (end 46.50 56.80) (width 0.30) (layer "B.Cu") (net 6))
 (segment (start 46.50 56.80) (end 46.50 23.81) (width 0.30) (layer "B.Cu") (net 6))
 (segment (start 46.50 23.81) (end 52.54 23.81) (width 0.30) (layer "B.Cu") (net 6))
 (segment (start 52.54 23.81) (end 52.54 25.08) (width 0.30) (layer "B.Cu") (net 6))
 (segment (start 6.50 42.86) (end 20.00 42.86) (width 0.30) (layer "B.Cu") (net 7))
 (segment (start 20.00 42.86) (end 20.00 57.60) (width 0.30) (layer "B.Cu") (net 7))
 (segment (start 20.00 57.60) (end 47.50 57.60) (width 0.30) (layer "B.Cu") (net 7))
 (segment (start 47.50 57.60) (end 47.50 27.62) (width 0.30) (layer "B.Cu") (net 7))
 (segment (start 47.50 27.62) (end 50.00 27.62) (width 0.30) (layer "B.Cu") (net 7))
 (segment (start 6.50 45.40) (end 22.00 45.40) (width 0.30) (layer "B.Cu") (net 8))
 (segment (start 22.00 45.40) (end 22.00 58.40) (width 0.30) (layer "B.Cu") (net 8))
 (segment (start 22.00 58.40) (end 48.50 58.40) (width 0.30) (layer "B.Cu") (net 8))
 (segment (start 48.50 58.40) (end 48.50 28.89) (width 0.30) (layer "B.Cu") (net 8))
 (segment (start 48.50 28.89) (end 52.54 28.89) (width 0.30) (layer "B.Cu") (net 8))
 (segment (start 52.54 28.89) (end 52.54 27.62) (width 0.30) (layer "B.Cu") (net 8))
 (segment (start 31.90 53.02) (end 35.00 53.02) (width 0.30) (layer "F.Cu") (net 3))
 (segment (start 35.00 53.02) (end 35.00 18.00) (width 0.30) (layer "F.Cu") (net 3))
 (segment (start 35.00 18.00) (end 41.27 18.00) (width 0.30) (layer "F.Cu") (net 3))
 (segment (start 41.27 18.00) (end 41.27 15.20) (width 0.30) (layer "F.Cu") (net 3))
 (segment (start 31.90 50.48) (end 36.20 50.48) (width 0.30) (layer "F.Cu") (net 4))
 (segment (start 36.20 50.48) (end 36.20 19.00) (width 0.30) (layer "F.Cu") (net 4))
 (segment (start 36.20 19.00) (end 43.81 19.00) (width 0.30) (layer "F.Cu") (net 4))
 (segment (start 43.81 19.00) (end 43.81 15.20) (width 0.30) (layer "F.Cu") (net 4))
 (segment (start 31.90 45.40) (end 38.73 45.40) (width 0.30) (layer "F.Cu") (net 16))
 (segment (start 38.73 45.40) (end 38.73 60.00) (width 0.30) (layer "F.Cu") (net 16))
 (segment (start 31.90 47.94) (end 36.19 47.94) (width 0.30) (layer "F.Cu") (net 17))
 (segment (start 36.19 47.94) (end 36.19 60.00) (width 0.30) (layer "F.Cu") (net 17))
 (segment (start 6.50 32.70) (end 16.00 32.70) (width 0.30) (layer "B.Cu") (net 5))
 (segment (start 16.00 32.70) (end 16.00 55.00) (width 0.30) (layer "B.Cu") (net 5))
 (segment (start 16.00 55.00) (end 22.00 60.00) (width 0.30) (layer "B.Cu") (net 5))
 (segment (start 22.00 60.00) (end 22.00 61.50) (width 0.30) (layer "B.Cu") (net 5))
 (segment (start 22.00 61.50) (end 43.81 61.50) (width 0.30) (layer "B.Cu") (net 5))
 (segment (start 43.81 61.50) (end 43.81 60.00) (width 0.30) (layer "B.Cu") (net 5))
 (segment (start 6.50 47.94) (end 4.50 47.94) (width 0.40) (layer "F.Cu") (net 9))
 (segment (start 4.50 47.94) (end 4.50 70.00) (width 0.40) (layer "F.Cu") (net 9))
 (segment (start 4.50 70.00) (end 12.19 70.00) (width 0.40) (layer "F.Cu") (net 9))
 (segment (start 19.81 70.00) (end 19.81 76.00) (width 0.40) (layer "F.Cu") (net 27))
 (segment (start 19.81 76.00) (end 19.81 84.00) (width 0.40) (layer "F.Cu") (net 27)))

